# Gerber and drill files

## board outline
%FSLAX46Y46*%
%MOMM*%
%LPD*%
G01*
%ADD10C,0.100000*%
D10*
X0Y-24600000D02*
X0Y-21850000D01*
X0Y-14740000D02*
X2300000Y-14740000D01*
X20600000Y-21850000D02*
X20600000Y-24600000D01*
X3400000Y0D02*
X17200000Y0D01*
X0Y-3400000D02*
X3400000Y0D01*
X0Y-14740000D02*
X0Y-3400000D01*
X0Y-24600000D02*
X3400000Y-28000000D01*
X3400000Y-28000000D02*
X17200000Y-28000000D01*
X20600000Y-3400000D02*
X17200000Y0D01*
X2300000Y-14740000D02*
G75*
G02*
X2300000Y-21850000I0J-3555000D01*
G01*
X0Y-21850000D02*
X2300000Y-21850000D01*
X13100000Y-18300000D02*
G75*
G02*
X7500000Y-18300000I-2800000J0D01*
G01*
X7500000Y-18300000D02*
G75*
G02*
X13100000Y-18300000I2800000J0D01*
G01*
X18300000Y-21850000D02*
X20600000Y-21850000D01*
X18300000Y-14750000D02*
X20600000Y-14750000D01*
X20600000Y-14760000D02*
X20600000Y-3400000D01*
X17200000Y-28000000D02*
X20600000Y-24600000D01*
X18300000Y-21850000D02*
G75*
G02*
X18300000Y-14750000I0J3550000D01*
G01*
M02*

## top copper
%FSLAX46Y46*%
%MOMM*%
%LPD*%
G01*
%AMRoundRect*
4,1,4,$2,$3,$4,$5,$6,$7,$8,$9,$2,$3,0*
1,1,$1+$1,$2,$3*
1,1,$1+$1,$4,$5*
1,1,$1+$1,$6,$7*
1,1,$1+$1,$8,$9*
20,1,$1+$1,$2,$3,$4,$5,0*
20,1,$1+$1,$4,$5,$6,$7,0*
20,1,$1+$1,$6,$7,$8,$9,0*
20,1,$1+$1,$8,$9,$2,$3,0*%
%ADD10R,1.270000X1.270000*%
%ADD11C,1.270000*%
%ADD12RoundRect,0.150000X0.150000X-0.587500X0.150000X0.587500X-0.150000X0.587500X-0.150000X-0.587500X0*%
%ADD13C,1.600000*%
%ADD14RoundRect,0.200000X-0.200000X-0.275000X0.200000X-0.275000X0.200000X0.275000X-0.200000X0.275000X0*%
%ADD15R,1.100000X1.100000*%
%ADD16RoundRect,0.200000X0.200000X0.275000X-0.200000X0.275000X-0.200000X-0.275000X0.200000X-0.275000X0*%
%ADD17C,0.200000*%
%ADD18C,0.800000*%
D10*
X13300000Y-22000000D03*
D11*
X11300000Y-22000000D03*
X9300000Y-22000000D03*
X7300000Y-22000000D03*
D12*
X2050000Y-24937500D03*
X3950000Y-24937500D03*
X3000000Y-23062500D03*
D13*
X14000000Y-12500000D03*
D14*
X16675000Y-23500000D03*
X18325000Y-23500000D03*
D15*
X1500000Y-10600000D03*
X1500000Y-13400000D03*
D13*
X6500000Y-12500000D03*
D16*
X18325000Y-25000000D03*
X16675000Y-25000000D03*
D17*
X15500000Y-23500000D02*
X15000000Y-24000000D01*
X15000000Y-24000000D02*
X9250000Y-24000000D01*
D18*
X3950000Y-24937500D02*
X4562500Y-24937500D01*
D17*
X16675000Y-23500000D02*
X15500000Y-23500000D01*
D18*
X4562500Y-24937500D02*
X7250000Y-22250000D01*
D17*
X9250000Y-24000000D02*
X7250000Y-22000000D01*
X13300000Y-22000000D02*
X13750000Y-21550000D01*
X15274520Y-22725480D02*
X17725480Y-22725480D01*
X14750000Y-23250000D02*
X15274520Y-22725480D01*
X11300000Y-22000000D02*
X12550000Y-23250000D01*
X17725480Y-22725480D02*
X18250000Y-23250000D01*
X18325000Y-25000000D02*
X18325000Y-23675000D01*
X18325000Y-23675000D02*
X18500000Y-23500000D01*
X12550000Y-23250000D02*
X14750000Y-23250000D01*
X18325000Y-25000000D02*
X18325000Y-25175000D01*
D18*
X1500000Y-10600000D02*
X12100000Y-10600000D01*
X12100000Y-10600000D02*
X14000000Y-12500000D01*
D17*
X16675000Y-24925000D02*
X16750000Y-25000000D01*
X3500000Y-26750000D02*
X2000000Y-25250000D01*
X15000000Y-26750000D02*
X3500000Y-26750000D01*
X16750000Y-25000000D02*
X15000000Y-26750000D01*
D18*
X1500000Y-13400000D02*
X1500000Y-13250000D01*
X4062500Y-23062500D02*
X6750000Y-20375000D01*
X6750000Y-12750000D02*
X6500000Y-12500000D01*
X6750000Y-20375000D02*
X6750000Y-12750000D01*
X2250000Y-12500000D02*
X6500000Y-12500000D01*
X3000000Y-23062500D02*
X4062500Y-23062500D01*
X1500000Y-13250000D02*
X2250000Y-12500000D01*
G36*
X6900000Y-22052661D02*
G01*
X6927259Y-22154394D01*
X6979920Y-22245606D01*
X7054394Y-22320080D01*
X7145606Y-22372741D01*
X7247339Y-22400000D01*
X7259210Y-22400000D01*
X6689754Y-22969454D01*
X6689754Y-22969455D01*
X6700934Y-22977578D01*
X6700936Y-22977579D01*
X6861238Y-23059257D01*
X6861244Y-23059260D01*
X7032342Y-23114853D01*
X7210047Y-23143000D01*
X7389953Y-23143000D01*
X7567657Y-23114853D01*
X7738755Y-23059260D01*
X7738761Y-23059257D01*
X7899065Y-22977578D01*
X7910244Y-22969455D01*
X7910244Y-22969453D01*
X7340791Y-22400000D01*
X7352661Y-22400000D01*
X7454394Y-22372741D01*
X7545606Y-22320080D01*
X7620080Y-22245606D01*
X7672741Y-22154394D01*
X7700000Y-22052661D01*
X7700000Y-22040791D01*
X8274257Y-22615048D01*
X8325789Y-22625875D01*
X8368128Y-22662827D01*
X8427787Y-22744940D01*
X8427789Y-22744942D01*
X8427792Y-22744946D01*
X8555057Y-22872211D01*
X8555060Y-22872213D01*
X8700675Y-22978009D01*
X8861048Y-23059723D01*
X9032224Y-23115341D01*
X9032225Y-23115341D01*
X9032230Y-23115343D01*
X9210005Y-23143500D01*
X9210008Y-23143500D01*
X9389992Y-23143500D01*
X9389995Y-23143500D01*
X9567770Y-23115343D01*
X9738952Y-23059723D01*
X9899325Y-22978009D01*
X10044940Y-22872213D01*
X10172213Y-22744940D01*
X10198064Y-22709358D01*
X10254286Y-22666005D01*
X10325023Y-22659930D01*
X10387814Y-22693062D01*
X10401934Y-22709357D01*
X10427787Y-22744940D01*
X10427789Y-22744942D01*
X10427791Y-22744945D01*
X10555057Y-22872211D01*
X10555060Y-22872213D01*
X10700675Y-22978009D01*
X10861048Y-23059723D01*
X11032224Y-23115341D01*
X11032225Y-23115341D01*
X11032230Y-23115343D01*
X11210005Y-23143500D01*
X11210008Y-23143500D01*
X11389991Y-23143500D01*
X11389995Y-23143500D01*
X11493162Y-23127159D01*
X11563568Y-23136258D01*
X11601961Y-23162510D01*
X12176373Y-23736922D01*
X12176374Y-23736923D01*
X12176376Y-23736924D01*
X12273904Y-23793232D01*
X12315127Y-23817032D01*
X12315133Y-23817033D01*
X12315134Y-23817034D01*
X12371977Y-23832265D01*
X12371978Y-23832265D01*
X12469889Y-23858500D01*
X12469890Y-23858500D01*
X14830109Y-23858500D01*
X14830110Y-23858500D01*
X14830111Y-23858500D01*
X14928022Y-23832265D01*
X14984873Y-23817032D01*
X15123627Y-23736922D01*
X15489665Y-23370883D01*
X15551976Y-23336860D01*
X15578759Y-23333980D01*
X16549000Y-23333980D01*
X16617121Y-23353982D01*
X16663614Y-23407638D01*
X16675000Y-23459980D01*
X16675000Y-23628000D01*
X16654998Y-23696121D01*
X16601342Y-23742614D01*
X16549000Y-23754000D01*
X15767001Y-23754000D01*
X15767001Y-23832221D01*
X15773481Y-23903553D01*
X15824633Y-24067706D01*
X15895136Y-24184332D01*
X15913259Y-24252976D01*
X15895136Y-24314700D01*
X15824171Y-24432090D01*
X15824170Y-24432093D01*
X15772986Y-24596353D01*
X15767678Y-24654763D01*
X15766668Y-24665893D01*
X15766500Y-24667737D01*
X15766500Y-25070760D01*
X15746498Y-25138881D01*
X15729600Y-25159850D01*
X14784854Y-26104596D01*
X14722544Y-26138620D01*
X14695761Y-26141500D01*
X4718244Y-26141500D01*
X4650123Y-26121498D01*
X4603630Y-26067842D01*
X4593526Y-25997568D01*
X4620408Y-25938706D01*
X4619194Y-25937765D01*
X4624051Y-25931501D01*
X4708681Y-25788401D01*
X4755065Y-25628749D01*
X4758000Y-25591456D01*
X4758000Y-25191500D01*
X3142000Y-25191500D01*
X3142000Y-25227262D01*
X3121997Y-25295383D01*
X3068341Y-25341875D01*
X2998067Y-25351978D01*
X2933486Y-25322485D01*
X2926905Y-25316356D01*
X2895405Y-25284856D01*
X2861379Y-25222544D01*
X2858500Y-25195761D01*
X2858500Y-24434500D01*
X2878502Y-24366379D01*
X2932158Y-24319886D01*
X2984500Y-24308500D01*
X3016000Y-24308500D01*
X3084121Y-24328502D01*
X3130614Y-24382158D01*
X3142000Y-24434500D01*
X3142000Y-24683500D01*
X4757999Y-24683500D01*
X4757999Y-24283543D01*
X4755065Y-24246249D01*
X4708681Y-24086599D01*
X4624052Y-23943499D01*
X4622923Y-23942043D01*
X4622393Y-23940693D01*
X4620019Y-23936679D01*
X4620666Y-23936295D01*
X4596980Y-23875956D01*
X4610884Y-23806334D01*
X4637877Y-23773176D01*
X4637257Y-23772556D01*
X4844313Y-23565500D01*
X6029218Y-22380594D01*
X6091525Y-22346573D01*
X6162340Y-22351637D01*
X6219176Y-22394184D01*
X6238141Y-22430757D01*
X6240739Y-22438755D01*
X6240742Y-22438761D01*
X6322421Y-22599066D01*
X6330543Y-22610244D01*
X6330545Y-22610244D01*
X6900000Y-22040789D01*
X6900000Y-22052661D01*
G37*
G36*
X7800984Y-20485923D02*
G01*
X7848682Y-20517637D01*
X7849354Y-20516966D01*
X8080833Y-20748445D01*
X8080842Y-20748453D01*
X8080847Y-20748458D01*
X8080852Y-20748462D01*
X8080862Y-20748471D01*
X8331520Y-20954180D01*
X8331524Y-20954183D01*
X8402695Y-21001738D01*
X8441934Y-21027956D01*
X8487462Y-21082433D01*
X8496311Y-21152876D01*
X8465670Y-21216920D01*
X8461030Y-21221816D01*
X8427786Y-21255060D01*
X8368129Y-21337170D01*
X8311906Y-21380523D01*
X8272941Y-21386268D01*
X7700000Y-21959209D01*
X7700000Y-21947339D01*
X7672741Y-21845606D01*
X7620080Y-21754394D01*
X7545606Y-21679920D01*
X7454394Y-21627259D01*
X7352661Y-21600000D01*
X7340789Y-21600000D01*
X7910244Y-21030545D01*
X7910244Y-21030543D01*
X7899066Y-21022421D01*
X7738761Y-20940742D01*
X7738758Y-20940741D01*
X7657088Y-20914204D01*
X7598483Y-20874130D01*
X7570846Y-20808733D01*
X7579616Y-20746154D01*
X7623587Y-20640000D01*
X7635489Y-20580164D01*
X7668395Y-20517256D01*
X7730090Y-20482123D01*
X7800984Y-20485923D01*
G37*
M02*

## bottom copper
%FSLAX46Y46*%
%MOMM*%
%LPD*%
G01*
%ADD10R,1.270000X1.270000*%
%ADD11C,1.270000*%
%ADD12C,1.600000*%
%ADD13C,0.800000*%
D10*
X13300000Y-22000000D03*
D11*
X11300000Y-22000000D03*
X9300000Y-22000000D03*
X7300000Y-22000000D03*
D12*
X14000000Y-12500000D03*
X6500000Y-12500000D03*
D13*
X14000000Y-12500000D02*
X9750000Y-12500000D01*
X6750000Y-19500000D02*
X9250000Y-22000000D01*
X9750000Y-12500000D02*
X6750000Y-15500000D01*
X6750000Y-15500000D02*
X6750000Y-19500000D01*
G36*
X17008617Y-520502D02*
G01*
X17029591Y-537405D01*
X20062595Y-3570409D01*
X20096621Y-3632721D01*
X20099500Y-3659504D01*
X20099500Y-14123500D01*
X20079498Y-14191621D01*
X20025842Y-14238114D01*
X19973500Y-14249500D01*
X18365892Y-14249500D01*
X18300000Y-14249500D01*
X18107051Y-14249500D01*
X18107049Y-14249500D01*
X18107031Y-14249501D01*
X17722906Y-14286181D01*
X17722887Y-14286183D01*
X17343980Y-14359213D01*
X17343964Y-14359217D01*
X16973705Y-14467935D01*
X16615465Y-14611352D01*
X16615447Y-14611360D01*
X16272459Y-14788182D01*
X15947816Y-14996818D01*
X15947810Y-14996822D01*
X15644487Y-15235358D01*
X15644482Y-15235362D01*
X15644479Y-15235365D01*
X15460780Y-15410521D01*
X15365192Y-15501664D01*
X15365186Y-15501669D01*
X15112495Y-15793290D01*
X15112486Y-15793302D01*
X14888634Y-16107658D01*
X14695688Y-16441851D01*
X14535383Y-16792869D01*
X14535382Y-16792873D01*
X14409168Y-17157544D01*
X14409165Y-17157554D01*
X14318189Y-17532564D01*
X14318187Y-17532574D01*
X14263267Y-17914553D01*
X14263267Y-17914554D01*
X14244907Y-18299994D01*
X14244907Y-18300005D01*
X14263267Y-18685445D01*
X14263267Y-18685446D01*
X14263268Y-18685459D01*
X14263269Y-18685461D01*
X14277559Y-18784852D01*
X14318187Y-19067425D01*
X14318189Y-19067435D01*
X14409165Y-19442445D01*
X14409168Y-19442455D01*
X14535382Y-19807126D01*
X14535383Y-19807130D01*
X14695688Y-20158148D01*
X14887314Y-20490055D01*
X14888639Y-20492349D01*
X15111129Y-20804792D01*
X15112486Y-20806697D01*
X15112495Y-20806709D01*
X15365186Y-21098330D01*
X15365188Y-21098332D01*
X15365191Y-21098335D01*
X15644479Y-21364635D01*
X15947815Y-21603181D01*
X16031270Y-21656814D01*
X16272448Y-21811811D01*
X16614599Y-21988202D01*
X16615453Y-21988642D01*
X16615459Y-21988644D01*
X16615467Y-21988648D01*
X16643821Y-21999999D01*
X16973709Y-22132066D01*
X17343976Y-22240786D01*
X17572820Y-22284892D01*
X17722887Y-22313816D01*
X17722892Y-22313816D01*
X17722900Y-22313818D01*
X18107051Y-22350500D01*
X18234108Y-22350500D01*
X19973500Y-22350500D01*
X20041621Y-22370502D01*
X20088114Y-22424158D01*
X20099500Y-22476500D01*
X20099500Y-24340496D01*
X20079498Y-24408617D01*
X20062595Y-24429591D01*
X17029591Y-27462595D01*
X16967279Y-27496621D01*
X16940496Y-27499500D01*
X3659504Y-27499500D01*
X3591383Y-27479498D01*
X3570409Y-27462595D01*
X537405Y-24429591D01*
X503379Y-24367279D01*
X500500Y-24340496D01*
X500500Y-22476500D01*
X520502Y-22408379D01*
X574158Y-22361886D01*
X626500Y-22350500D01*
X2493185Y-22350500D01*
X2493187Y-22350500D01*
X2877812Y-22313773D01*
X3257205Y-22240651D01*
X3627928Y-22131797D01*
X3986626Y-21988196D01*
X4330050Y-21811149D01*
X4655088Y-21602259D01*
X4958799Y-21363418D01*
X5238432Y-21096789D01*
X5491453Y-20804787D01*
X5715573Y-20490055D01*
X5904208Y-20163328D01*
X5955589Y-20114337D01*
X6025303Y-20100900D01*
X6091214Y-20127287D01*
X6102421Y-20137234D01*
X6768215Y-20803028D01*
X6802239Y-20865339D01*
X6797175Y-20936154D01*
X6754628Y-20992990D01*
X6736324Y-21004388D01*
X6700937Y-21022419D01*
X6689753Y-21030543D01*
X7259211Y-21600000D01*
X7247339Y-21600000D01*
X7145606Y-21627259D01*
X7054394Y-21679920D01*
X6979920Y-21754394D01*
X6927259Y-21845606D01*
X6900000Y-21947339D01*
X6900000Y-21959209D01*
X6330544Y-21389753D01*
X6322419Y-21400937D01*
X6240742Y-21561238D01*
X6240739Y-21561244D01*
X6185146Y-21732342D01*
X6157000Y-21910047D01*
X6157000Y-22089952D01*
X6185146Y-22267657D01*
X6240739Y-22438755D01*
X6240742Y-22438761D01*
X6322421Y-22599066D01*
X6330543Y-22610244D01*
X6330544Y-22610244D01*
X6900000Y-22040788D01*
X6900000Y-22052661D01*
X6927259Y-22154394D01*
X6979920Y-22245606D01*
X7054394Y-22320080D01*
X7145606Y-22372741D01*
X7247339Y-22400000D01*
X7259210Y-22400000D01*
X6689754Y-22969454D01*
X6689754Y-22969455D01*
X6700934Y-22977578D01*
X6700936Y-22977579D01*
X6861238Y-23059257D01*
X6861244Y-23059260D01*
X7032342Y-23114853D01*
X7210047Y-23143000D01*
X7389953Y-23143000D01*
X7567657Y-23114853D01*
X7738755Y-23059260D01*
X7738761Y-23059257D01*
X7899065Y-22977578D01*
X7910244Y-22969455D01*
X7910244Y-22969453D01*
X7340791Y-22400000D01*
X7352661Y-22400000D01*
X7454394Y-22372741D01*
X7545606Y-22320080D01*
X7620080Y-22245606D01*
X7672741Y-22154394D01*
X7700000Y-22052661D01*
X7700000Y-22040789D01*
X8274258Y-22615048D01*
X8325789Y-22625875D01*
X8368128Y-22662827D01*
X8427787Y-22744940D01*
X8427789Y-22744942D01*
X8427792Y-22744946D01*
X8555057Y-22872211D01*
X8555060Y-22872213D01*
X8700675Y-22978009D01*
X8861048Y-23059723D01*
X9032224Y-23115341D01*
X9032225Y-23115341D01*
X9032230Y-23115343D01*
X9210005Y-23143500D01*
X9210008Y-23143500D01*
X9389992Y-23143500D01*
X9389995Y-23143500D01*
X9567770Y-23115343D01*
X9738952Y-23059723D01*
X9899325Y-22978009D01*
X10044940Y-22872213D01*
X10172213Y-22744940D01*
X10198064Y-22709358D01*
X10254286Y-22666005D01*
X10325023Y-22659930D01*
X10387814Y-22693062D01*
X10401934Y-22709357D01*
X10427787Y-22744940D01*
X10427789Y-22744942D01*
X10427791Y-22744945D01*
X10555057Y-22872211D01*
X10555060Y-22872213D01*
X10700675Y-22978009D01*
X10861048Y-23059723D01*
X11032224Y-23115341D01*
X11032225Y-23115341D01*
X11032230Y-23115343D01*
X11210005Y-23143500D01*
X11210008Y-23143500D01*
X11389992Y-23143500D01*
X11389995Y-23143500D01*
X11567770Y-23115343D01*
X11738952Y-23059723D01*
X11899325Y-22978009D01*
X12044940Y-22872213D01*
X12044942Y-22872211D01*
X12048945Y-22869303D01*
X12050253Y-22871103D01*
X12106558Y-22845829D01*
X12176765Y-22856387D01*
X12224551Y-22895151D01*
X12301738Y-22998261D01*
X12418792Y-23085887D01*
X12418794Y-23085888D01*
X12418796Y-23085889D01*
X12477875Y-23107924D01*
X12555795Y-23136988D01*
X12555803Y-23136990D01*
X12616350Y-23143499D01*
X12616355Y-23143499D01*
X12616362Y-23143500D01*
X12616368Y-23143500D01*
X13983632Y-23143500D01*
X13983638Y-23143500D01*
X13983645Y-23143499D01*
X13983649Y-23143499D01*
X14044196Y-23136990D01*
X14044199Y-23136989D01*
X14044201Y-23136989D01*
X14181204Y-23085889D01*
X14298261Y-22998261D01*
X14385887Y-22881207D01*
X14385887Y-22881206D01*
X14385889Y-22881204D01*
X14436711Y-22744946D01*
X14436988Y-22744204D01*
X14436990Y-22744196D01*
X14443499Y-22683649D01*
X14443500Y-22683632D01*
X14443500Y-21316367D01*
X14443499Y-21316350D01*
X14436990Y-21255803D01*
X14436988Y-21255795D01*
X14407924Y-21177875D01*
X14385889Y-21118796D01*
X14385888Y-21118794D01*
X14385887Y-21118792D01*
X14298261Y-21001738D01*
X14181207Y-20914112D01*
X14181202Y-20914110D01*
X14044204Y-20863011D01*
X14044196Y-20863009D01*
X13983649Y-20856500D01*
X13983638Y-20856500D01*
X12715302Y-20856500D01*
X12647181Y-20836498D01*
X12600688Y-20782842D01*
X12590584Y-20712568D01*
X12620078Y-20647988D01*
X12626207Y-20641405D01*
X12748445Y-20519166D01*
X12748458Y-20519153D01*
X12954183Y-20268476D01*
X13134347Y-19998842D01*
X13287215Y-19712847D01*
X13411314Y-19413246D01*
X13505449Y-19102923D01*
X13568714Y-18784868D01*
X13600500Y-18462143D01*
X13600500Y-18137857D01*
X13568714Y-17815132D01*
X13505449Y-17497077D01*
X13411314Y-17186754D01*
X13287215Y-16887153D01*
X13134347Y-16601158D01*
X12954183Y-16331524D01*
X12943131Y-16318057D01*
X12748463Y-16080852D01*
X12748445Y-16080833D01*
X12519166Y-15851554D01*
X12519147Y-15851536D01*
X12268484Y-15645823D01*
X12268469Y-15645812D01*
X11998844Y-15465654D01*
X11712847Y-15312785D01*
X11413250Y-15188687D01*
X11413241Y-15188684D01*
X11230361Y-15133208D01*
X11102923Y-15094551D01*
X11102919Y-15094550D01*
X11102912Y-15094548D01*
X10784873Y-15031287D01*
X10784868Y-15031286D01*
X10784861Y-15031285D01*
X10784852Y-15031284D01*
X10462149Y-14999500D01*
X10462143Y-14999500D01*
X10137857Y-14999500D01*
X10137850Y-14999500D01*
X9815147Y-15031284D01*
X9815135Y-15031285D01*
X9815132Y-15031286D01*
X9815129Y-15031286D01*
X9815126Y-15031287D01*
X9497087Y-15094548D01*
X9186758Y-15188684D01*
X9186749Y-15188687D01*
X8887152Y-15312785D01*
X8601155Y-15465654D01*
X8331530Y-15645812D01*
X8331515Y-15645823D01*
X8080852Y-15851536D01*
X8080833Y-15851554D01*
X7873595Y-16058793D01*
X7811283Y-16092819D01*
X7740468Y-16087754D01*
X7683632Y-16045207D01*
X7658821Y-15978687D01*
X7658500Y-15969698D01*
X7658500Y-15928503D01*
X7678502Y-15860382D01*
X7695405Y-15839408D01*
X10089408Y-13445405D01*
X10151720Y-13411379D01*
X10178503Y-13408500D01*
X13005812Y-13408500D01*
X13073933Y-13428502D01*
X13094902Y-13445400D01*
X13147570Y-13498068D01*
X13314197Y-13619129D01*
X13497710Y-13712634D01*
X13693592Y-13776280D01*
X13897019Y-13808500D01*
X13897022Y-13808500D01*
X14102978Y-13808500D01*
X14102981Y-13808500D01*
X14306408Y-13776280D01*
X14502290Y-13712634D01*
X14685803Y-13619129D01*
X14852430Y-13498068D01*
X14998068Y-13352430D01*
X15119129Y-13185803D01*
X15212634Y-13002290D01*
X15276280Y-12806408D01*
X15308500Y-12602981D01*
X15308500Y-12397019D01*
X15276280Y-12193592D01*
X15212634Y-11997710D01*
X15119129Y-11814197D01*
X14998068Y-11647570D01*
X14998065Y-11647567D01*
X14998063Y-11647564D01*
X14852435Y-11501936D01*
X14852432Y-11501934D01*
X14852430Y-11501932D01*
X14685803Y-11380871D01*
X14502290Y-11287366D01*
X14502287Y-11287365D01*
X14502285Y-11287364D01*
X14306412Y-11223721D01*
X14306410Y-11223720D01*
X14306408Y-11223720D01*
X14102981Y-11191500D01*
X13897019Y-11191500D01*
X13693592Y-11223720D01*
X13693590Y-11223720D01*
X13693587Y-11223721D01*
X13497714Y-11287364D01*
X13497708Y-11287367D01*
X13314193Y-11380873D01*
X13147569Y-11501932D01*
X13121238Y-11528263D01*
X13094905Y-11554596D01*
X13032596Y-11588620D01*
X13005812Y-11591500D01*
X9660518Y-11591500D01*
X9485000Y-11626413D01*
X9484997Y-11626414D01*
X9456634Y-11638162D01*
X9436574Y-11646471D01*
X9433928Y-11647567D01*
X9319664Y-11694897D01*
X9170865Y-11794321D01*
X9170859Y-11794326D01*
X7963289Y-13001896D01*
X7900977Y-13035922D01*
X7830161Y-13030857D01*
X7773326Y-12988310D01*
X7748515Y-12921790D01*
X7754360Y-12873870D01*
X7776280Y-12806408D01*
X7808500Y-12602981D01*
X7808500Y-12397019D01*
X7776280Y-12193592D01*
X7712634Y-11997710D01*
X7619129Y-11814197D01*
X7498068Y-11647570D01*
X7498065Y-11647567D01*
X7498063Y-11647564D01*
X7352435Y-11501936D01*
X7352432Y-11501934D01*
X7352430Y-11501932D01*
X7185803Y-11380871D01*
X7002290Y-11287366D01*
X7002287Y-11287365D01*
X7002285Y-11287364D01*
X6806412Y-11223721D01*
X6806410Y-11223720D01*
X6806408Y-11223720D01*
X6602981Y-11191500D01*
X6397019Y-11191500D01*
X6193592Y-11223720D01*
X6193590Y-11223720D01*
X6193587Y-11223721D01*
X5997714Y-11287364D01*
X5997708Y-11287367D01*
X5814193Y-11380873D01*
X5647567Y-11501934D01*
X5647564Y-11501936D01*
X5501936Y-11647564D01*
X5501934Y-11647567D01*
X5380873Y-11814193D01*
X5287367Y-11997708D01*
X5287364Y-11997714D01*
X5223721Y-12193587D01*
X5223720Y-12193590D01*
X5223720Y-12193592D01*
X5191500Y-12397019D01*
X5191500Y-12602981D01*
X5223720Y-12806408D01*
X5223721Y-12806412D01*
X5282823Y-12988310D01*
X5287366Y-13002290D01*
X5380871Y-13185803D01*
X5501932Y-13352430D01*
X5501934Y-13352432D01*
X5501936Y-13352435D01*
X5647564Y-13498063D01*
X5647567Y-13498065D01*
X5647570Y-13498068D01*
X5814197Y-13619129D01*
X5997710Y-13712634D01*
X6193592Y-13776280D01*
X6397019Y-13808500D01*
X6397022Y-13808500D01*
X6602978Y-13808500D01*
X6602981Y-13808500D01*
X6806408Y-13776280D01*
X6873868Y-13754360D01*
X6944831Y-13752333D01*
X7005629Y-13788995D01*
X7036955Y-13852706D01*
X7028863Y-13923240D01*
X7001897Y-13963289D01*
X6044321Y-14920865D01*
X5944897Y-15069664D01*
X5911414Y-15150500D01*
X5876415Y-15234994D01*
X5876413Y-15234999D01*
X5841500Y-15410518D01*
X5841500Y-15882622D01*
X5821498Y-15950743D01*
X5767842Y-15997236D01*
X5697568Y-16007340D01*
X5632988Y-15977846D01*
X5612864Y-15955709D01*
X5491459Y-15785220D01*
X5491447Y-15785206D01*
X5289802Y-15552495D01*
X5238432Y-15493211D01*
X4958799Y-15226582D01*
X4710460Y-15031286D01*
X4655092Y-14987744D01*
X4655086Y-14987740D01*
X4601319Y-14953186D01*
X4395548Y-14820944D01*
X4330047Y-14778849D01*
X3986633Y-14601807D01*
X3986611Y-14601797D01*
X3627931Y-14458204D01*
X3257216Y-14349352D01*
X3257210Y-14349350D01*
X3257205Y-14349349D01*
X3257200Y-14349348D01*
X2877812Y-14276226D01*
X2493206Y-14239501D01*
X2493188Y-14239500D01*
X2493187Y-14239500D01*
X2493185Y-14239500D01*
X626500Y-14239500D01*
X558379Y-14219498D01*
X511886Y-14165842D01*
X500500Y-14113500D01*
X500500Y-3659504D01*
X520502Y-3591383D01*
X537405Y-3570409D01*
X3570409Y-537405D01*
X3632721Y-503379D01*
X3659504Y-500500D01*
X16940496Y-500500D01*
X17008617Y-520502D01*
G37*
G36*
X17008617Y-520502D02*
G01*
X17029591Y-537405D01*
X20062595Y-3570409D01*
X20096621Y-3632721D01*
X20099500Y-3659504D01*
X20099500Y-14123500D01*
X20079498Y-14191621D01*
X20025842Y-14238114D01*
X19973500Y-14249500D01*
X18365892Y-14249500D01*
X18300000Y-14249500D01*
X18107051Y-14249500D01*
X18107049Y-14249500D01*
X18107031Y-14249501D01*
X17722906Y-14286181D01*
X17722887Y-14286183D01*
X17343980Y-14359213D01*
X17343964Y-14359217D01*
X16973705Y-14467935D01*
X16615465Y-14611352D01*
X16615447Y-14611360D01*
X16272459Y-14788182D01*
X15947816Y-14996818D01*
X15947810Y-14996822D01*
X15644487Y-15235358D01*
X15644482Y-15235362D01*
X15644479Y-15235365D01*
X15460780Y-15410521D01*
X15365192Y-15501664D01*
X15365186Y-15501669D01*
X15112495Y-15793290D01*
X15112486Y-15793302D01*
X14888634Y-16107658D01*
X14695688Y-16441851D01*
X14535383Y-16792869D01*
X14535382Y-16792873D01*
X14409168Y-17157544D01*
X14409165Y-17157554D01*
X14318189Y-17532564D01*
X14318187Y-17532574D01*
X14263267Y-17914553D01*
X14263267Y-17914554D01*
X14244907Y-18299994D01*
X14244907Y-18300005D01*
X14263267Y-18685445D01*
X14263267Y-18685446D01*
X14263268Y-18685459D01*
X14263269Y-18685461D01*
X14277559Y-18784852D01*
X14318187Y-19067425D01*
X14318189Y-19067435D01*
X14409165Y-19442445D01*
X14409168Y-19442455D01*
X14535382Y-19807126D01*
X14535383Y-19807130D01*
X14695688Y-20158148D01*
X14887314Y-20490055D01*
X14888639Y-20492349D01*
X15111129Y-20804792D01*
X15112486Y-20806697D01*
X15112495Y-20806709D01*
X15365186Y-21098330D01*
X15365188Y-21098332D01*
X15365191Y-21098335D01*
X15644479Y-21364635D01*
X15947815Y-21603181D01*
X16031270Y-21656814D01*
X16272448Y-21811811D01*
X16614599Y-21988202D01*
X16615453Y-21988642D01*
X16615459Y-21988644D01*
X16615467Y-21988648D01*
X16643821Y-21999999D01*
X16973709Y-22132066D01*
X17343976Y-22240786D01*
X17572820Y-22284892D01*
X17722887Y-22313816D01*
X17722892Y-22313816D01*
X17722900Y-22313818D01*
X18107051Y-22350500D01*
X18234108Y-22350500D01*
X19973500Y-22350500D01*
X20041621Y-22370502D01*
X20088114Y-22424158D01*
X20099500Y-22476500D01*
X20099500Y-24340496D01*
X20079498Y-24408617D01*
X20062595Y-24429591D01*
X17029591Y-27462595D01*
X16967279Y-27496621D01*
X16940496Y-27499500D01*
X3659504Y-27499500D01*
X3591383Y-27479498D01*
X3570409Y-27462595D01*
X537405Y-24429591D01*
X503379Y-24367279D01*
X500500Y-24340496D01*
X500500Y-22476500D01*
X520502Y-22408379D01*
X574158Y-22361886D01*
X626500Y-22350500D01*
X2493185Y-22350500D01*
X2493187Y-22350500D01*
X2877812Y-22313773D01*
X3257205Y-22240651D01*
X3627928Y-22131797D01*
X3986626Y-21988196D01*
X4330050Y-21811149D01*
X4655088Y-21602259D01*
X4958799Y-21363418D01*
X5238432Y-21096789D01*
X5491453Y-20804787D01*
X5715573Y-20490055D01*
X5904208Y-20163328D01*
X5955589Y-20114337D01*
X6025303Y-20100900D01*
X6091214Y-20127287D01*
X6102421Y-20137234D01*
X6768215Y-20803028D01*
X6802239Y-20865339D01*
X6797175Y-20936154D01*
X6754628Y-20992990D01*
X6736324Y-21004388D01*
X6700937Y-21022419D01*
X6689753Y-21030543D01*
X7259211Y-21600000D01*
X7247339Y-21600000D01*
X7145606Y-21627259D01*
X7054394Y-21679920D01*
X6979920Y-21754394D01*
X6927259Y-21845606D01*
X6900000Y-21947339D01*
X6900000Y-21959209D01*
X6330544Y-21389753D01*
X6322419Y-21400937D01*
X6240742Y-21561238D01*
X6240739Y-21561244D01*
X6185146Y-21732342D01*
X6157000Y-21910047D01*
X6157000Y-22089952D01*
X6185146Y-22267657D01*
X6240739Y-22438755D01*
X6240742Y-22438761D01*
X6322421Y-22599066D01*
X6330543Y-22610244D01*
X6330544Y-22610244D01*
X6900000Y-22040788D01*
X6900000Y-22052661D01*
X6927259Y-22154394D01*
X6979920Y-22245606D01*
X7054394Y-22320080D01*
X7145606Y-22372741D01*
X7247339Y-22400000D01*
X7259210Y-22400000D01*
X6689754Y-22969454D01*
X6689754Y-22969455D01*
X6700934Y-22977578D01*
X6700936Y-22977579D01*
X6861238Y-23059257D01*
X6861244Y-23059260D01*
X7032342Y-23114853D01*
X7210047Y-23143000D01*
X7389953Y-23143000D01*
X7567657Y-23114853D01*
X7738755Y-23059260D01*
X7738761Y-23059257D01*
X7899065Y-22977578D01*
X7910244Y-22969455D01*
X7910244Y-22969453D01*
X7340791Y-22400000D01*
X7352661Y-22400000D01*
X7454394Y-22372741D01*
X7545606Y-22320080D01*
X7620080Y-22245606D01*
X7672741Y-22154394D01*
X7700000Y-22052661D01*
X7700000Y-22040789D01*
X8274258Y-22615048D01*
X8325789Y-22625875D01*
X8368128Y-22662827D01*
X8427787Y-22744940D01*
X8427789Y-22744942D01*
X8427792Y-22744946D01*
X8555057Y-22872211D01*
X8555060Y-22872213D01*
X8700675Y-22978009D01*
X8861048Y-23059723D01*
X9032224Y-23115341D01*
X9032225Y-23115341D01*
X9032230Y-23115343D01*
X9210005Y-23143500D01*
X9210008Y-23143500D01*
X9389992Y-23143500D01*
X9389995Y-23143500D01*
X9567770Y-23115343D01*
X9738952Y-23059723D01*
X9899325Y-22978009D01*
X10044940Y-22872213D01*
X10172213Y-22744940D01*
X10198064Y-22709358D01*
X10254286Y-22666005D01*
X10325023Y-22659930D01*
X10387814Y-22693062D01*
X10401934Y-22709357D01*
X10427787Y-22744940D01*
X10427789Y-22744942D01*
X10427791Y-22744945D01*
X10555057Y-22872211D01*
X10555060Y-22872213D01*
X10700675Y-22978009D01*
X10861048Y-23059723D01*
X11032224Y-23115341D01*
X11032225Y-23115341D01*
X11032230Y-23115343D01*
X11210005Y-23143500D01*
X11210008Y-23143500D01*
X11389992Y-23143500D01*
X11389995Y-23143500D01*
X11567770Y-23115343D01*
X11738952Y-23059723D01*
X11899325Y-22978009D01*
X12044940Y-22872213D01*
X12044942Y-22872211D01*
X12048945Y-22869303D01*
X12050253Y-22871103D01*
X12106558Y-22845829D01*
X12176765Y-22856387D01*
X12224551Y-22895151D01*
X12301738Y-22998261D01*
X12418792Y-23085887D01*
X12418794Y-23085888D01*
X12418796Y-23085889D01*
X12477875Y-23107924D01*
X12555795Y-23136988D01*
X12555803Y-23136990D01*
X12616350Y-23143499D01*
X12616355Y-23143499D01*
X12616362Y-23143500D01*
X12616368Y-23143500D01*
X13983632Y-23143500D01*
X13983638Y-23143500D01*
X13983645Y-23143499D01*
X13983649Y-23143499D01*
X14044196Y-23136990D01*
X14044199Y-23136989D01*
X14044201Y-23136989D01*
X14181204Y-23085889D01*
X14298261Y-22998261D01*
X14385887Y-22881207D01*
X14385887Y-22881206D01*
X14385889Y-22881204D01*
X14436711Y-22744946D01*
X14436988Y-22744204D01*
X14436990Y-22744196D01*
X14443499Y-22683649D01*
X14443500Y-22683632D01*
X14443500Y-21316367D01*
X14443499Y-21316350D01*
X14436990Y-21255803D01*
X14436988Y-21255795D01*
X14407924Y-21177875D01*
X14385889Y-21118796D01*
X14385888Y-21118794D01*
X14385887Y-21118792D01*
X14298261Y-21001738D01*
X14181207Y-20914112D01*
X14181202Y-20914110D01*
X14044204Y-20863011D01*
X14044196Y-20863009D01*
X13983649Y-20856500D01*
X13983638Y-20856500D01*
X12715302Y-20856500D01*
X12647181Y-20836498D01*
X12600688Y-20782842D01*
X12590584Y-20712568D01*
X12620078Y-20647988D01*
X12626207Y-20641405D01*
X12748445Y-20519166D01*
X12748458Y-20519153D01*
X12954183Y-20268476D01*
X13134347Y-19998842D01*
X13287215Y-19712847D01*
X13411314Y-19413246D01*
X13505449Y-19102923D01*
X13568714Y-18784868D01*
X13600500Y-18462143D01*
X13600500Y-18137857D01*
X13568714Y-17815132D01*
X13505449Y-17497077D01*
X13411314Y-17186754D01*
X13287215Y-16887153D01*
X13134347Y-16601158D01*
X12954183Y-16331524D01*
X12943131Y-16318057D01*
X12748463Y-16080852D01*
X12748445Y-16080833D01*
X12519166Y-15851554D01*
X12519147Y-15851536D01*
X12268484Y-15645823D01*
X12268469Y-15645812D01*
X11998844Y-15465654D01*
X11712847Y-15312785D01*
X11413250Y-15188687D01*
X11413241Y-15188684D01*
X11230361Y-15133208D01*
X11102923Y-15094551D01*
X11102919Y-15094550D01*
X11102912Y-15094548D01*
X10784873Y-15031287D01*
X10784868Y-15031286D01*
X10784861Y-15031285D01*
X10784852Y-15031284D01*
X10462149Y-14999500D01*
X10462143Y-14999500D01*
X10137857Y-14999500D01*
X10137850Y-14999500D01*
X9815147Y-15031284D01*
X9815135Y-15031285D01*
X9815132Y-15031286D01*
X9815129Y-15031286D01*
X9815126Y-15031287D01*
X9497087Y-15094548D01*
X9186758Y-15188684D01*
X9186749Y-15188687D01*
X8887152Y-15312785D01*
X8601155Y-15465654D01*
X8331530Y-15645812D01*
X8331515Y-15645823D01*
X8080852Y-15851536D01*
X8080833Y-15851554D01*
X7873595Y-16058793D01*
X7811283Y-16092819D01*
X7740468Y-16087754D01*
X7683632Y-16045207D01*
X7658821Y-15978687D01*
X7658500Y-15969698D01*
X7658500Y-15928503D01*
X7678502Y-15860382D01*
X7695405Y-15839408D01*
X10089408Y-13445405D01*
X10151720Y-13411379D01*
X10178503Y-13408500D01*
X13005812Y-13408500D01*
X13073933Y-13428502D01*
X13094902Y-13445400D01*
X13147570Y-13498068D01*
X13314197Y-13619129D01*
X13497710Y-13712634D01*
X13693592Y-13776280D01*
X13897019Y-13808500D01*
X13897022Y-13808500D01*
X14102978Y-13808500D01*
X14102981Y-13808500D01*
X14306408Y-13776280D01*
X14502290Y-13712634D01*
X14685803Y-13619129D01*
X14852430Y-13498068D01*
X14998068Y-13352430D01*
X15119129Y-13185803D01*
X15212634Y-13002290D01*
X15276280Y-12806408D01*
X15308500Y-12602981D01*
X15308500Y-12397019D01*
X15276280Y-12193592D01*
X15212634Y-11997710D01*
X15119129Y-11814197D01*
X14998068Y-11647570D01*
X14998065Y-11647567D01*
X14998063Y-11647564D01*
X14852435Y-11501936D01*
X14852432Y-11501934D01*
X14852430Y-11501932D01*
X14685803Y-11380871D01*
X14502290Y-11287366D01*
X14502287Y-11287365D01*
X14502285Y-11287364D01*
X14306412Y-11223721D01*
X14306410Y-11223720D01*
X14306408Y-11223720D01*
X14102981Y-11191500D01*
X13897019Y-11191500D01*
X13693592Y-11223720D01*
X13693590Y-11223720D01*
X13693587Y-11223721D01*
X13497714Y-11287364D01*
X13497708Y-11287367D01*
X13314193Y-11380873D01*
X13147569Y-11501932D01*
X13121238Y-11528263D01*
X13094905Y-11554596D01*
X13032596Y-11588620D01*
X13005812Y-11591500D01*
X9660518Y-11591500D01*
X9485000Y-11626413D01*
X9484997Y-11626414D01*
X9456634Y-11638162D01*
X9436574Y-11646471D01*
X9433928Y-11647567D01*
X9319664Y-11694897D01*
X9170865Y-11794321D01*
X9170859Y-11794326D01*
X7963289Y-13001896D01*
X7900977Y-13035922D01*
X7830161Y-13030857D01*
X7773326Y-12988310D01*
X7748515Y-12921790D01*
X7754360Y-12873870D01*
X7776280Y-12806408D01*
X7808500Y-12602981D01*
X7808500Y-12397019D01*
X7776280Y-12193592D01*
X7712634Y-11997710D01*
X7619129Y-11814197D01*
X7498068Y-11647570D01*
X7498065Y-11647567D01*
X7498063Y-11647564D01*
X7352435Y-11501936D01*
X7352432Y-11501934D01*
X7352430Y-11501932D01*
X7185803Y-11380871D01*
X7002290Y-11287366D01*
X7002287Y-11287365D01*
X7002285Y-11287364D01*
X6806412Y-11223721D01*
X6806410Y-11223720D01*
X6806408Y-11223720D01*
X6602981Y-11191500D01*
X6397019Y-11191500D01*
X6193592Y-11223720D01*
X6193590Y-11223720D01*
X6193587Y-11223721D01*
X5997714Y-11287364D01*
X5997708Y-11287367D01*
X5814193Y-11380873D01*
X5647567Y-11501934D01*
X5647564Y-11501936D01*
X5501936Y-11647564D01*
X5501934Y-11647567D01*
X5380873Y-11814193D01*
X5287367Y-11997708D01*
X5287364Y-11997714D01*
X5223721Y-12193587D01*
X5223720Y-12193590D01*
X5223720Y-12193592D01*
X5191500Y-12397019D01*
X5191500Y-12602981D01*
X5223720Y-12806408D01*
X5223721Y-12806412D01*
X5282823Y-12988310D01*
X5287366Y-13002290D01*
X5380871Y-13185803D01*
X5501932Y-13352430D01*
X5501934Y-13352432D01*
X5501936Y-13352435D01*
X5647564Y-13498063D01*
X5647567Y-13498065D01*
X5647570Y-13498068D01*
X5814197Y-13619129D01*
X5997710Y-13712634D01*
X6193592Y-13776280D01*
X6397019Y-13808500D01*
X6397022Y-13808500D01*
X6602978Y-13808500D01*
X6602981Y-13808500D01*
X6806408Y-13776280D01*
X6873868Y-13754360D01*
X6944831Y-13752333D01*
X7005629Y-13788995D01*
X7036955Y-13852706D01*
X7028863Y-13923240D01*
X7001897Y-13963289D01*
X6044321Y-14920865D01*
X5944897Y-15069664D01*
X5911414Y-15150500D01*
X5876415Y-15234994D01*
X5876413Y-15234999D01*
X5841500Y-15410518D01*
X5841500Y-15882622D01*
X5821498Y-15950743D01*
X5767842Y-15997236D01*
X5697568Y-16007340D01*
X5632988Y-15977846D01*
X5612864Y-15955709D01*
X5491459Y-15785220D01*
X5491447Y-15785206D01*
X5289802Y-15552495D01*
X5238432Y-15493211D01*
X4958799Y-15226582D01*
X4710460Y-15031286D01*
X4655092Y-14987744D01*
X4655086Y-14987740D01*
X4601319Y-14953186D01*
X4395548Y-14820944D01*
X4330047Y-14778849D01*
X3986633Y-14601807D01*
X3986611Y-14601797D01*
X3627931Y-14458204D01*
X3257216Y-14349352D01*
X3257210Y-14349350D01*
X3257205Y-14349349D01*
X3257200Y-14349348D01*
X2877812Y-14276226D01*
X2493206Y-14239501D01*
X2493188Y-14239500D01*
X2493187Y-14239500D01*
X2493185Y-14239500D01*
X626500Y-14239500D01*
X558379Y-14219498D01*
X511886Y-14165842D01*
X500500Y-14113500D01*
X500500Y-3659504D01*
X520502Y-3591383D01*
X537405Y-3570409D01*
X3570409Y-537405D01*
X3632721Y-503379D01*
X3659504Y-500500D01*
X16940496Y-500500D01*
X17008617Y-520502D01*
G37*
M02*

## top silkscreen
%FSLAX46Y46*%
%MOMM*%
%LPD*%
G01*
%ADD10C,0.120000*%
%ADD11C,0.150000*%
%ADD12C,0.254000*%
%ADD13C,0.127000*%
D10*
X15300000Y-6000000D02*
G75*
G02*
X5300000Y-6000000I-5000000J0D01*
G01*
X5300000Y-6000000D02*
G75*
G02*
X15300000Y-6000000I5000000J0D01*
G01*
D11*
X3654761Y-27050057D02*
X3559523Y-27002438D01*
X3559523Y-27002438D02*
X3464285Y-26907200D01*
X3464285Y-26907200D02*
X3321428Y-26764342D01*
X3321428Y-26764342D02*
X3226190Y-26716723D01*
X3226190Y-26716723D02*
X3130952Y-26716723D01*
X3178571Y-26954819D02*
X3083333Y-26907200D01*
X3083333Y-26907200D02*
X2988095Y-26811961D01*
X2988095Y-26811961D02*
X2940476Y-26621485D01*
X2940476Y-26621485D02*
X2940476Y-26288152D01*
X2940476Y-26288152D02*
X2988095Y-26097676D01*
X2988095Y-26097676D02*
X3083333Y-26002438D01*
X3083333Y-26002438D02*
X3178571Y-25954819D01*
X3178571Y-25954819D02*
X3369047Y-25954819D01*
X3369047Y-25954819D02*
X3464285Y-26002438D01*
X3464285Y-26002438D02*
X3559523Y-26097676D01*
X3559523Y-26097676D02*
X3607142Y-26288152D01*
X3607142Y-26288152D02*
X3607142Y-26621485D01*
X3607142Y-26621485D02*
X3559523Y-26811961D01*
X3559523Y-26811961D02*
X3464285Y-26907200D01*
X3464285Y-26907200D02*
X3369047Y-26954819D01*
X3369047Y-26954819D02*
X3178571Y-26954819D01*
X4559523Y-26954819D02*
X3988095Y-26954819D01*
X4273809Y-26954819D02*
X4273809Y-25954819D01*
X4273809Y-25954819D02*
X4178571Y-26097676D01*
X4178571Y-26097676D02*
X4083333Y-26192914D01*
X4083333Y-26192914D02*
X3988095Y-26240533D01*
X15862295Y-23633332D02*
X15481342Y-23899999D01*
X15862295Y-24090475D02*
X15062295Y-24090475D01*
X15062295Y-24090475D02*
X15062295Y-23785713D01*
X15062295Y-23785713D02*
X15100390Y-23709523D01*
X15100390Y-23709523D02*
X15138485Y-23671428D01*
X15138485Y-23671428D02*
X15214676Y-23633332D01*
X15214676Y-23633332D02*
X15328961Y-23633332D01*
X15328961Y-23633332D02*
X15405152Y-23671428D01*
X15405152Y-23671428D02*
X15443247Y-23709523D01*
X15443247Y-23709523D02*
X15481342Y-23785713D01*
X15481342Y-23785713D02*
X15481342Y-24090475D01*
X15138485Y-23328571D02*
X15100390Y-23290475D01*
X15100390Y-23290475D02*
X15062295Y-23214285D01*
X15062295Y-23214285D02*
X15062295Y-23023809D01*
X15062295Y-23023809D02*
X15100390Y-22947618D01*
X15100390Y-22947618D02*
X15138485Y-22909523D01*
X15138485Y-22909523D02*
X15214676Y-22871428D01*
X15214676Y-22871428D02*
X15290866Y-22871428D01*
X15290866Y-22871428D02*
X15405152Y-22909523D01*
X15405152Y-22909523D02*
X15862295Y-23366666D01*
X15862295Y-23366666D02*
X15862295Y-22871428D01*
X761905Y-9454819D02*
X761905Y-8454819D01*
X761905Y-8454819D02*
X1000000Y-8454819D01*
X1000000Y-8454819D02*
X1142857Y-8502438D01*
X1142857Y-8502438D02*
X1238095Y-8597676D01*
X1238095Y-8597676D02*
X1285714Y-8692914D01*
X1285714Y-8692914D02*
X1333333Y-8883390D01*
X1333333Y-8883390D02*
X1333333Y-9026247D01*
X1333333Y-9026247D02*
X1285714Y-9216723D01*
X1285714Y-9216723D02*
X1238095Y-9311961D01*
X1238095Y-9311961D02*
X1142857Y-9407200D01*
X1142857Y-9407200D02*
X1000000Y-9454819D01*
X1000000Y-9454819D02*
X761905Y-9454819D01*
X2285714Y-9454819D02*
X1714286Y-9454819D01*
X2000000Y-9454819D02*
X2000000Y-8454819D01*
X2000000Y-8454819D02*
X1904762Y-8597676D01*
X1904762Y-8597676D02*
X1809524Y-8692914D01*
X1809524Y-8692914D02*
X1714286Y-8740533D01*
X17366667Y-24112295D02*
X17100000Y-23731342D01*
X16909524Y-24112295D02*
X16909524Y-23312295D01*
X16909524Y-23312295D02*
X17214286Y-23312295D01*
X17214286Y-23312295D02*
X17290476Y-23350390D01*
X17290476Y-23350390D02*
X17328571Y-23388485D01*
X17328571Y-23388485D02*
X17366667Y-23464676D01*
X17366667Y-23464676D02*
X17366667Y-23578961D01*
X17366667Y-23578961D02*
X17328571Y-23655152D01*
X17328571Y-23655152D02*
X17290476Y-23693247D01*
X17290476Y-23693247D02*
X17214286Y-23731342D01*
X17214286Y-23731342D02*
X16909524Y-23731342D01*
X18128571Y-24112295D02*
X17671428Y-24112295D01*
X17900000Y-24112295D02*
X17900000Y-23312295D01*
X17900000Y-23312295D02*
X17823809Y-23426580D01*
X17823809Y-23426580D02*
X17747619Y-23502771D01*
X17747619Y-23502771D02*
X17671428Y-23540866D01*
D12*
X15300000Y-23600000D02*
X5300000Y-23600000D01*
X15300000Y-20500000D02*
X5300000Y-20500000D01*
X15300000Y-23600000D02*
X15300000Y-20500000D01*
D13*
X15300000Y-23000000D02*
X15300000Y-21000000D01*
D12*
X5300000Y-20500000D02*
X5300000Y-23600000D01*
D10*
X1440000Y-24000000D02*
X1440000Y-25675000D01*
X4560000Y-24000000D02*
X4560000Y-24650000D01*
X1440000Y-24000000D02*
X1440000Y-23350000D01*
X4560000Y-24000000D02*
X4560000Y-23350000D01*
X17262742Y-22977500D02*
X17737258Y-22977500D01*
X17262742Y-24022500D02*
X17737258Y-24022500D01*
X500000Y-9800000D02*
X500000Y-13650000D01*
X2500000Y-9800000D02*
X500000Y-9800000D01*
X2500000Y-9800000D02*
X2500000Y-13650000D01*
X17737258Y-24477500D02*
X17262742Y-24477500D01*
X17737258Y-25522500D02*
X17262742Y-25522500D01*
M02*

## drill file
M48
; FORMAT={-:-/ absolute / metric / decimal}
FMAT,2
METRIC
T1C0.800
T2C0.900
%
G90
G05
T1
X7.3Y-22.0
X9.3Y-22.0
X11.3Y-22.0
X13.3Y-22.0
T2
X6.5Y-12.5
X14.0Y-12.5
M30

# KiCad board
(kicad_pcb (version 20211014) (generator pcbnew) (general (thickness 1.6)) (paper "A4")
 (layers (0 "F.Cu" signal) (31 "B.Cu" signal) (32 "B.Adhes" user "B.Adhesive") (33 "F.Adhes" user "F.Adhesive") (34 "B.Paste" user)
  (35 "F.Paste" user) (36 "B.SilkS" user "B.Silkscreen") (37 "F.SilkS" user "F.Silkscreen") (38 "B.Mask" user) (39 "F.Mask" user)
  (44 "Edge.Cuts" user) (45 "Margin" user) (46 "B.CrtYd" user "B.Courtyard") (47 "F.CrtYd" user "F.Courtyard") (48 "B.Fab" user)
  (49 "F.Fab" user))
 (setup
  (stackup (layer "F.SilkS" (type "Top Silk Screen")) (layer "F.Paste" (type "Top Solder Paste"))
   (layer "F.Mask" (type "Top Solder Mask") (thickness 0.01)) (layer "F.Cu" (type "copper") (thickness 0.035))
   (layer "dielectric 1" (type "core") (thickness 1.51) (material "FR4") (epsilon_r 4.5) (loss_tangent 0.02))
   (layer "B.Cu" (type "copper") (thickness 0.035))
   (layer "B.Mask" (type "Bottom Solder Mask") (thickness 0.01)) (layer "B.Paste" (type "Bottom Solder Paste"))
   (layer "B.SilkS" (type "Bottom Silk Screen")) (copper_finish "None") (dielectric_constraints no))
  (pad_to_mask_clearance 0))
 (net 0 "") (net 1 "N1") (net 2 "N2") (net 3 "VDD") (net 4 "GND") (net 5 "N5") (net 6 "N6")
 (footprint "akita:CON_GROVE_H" (layer "F.Cu") (at 10.3 22 180)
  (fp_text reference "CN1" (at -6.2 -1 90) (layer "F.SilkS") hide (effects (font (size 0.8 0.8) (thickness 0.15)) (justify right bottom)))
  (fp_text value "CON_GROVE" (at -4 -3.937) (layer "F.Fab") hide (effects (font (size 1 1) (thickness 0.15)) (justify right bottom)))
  (fp_line (start -5 -1.6) (end 5 -1.6) (layer "F.SilkS") (width 0.254))
  (fp_line (start -5 1.5) (end 5 1.5) (layer "F.SilkS") (width 0.254))
  (fp_line (start -5 -1.6) (end -5 1.5) (layer "F.SilkS") (width 0.254))
  (fp_line (start -5 -1) (end -5 1) (layer "F.SilkS") (width 0.127))
  (fp_line (start 5 1.5) (end 5 -1.6) (layer "F.SilkS") (width 0.254))
  (pad "1" thru_hole rect (at -3 0 180) (size 1.27 1.27) (drill 0.8) (layers *.Cu *.Mask) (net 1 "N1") (solder_mask_margin 0.1016))
  (pad "2" thru_hole circle (at -1 0 180) (size 1.27 1.27) (drill 0.8) (layers *.Cu *.Mask) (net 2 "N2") (solder_mask_margin 0.1016))
  (pad "3" thru_hole circle (at 1 0 180) (size 1.27 1.27) (drill 0.8) (layers *.Cu *.Mask) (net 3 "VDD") (solder_mask_margin 0.1016))
  (pad "4" thru_hole circle (at 3 0 180) (size 1.27 1.27) (drill 0.8) (layers *.Cu *.Mask) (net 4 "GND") (solder_mask_margin 0.1016)))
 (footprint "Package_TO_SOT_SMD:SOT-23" (layer "F.Cu") (at 3 24 90)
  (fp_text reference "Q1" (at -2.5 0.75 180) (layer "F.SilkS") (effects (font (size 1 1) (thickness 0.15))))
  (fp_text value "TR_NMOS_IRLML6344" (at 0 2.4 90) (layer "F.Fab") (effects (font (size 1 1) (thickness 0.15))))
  (fp_line (start 0 -1.56) (end -1.675 -1.56) (layer "F.SilkS") (width 0.12))
  (fp_line (start 0 1.56) (end -0.65 1.56) (layer "F.SilkS") (width 0.12))
  (fp_line (start 0 -1.56) (end 0.65 -1.56) (layer "F.SilkS") (width 0.12))
  (fp_line (start 0 1.56) (end 0.65 1.56) (layer "F.SilkS") (width 0.12))
  (pad "1" smd roundrect locked (at -0.9375 -0.95 90) (size 1.475 0.6) (layers "F.Cu" "F.Paste" "F.Mask") (roundrect_rratio 0.25)
   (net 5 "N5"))
  (pad "2" smd roundrect locked (at -0.9375 0.95 90) (size 1.475 0.6) (layers "F.Cu" "F.Paste" "F.Mask") (roundrect_rratio 0.25)
   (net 4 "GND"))
  (pad "3" smd roundrect locked (at 0.9375 0 90) (size 1.475 0.6) (layers "F.Cu" "F.Paste" "F.Mask") (roundrect_rratio 0.25) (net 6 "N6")))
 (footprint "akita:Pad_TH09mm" (layer "F.Cu") (at 14 12.5 11)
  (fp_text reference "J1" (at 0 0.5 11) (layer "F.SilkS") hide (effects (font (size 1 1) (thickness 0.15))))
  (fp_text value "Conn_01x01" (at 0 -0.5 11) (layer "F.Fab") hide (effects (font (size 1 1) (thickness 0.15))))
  (pad "1" thru_hole circle locked (at 0 0 11) (size 1.6 1.6) (drill 0.9) (layers *.Cu *.Mask) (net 3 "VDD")))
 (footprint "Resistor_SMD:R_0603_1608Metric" (layer "F.Cu") (at 17.5 23.5)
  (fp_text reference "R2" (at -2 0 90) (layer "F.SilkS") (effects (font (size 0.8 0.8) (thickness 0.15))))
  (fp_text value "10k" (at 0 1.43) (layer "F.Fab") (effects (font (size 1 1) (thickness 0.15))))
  (fp_line (start -0.237258 -0.5225) (end 0.237258 -0.5225) (layer "F.SilkS") (width 0.12))
  (fp_line (start -0.237258 0.5225) (end 0.237258 0.5225) (layer "F.SilkS") (width 0.12))
  (pad "1" smd roundrect locked (at -0.825 0) (size 0.8 0.95) (layers "F.Cu" "F.Paste" "F.Mask") (roundrect_rratio 0.25) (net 4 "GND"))
  (pad "2" smd roundrect locked (at 0.825 0) (size 0.8 0.95) (layers "F.Cu" "F.Paste" "F.Mask") (roundrect_rratio 0.25) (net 2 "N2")))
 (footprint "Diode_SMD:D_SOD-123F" (layer "F.Cu") (at 1.5 12 -90)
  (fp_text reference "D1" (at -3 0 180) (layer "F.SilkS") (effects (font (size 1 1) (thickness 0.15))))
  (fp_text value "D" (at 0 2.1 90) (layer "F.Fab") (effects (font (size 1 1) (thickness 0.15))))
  (fp_line (start -2.2 1) (end 1.65 1) (layer "F.SilkS") (width 0.12))
  (fp_line (start -2.2 -1) (end -2.2 1) (layer "F.SilkS") (width 0.12))
  (fp_line (start -2.2 -1) (end 1.65 -1) (layer "F.SilkS") (width 0.12))
  (pad "1" smd rect locked (at -1.4 0 270) (size 1.1 1.1) (layers "F.Cu" "F.Paste" "F.Mask") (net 3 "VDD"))
  (pad "2" smd rect locked (at 1.4 0 270) (size 1.1 1.1) (layers "F.Cu" "F.Paste" "F.Mask") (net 6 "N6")))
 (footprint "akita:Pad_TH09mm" (layer "F.Cu") (at 6.5 12.5)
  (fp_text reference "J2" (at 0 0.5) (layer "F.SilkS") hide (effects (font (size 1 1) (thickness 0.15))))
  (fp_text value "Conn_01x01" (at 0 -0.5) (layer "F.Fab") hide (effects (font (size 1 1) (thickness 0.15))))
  (pad "1" thru_hole circle locked (at 0 0) (size 1.6 1.6) (drill 0.9) (layers *.Cu *.Mask) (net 6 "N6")))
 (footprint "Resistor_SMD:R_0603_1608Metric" (layer "F.Cu") (at 17.5 25 180)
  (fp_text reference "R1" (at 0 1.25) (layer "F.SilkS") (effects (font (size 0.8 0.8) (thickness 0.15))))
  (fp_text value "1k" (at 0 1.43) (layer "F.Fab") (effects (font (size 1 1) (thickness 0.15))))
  (fp_line (start -0.237258 0.5225) (end 0.237258 0.5225) (layer "F.SilkS") (width 0.12))
  (fp_line (start -0.237258 -0.5225) (end 0.237258 -0.5225) (layer "F.SilkS") (width 0.12))
  (pad "1" smd roundrect locked (at -0.825 0 180) (size 0.8 0.95) (layers "F.Cu" "F.Paste" "F.Mask") (roundrect_rratio 0.25) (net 2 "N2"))
  (pad "2" smd roundrect locked (at 0.825 0 180) (size 0.8 0.95) (layers "F.Cu" "F.Paste" "F.Mask") (roundrect_rratio 0.25) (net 5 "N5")))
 (gr_circle (center 10.3 6) (end 15.3 6) (layer "F.SilkS") (width 0.12) (fill none))
 (gr_line (start 0 24.6) (end 0 21.85) (layer "Edge.Cuts") (width 0.1))
 (gr_line (start 0 14.74) (end 2.3 14.74) (layer "Edge.Cuts") (width 0.1))
 (gr_line (start 20.6 21.85) (end 20.6 24.6) (layer "Edge.Cuts") (width 0.1))
 (gr_line (start 3.4 0) (end 17.2 0) (layer "Edge.Cuts") (width 0.1))
 (gr_line (start 0 3.4) (end 3.4 0) (layer "Edge.Cuts") (width 0.1))
 (gr_line (start 0 14.74) (end 0 3.4) (layer "Edge.Cuts") (width 0.1))
 (gr_line (start 0 24.6) (end 3.4 28) (layer "Edge.Cuts") (width 0.1))
 (gr_line (start 3.4 28) (end 17.2 28) (layer "Edge.Cuts") (width 0.1))
 (gr_line (start 20.6 3.4) (end 17.2 0) (layer "Edge.Cuts") (width 0.1))
 (gr_arc (start 2.3 14.74) (mid 5.855 18.295) (end 2.3 21.85) (layer "Edge.Cuts") (width 0.1))
 (gr_line (start 0 21.85) (end 2.3 21.85) (layer "Edge.Cuts") (width 0.1))
 (gr_circle (center 10.3 18.3) (end 13.1 18.3) (layer "Edge.Cuts") (width 0.1) (fill none))
 (gr_line (start 18.3 21.85) (end 20.6 21.85) (layer "Edge.Cuts") (width 0.1))
 (gr_line (start 18.3 14.75) (end 20.6 14.75) (layer "Edge.Cuts") (width 0.1))
 (gr_line (start 20.6 14.76) (end 20.6 3.4) (layer "Edge.Cuts") (width 0.1))
 (gr_line (start 17.2 28) (end 20.6 24.6) (layer "Edge.Cuts") (width 0.1))
 (gr_arc (start 18.3 21.85) (mid 14.75 18.3) (end 18.3 14.75) (layer "Edge.Cuts") (width 0.1))
 (segment (start 15.5 23.5) (end 15 24) (width 0.2) (layer "F.Cu") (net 4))
 (segment (start 15 24) (end 9.25 24) (width 0.2) (layer "F.Cu") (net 4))
 (segment (start 3.95 24.9375) (end 4.5625 24.9375) (width 0.8) (layer "F.Cu") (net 4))
 (segment (start 16.675 23.5) (end 15.5 23.5) (width 0.2) (layer "F.Cu") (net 4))
 (segment (start 4.5625 24.9375) (end 7.25 22.25) (width 0.8) (layer "F.Cu") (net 4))
 (segment (start 9.25 24) (end 7.25 22) (width 0.2) (layer "F.Cu") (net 4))
 (segment (start 13.3 22) (end 13.75 21.55) (width 0.2) (layer "F.Cu") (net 1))
 (segment (start 15.27452 22.72548) (end 17.72548 22.72548) (width 0.2) (layer "F.Cu") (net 2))
 (segment (start 14.75 23.25) (end 15.27452 22.72548) (width 0.2) (layer "F.Cu") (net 2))
 (segment (start 11.3 22) (end 12.55 23.25) (width 0.2) (layer "F.Cu") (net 2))
 (segment (start 17.72548 22.72548) (end 18.25 23.25) (width 0.2) (layer "F.Cu") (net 2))
 (segment (start 18.325 25) (end 18.325 23.675) (width 0.2) (layer "F.Cu") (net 2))
 (segment (start 18.325 23.675) (end 18.5 23.5) (width 0.2) (layer "F.Cu") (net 2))
 (segment (start 12.55 23.25) (end 14.75 23.25) (width 0.2) (layer "F.Cu") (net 2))
 (segment (start 18.325 25) (end 18.325 25.175) (width 0.2) (layer "F.Cu") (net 2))
 (segment (start 1.5 10.6) (end 12.1 10.6) (width 0.8) (layer "F.Cu") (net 3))
 (segment (start 12.1 10.6) (end 14 12.5) (width 0.8) (layer "F.Cu") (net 3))
 (segment (start 14 12.5) (end 9.75 12.5) (width 0.8) (layer "B.Cu") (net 3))
 (segment (start 6.75 19.5) (end 9.25 22) (width 0.8) (layer "B.Cu") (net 3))
 (segment (start 9.75 12.5) (end 6.75 15.5) (width 0.8) (layer "B.Cu") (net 3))
 (segment (start 6.75 15.5) (end 6.75 19.5) (width 0.8) (layer "B.Cu") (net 3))
 (segment (start 16.675 24.925) (end 16.75 25) (width 0.2) (layer "F.Cu") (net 5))
 (segment (start 3.5 26.75) (end 2 25.25) (width 0.2) (layer "F.Cu") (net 5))
 (segment (start 15 26.75) (end 3.5 26.75) (width 0.2) (layer "F.Cu") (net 5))
 (segment (start 16.75 25) (end 15 26.75) (width 0.2) (layer "F.Cu") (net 5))
 (segment (start 1.5 13.4) (end 1.5 13.25) (width 0.8) (layer "F.Cu") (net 6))
 (segment (start 4.0625 23.0625) (end 6.75 20.375) (width 0.8) (layer "F.Cu") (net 6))
 (segment (start 6.75 12.75) (end 6.5 12.5) (width 0.8) (layer "F.Cu") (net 6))
 (segment (start 6.75 20.375) (end 6.75 12.75) (width 0.8) (layer "F.Cu") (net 6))
 (segment (start 2.25 12.5) (end 6.5 12.5) (width 0.8) (layer "F.Cu") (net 6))
 (segment (start 3 23.0625) (end 4.0625 23.0625) (width 0.8) (layer "F.Cu") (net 6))
 (segment (start 1.5 13.25) (end 2.25 12.5) (width 0.8) (layer "F.Cu") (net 6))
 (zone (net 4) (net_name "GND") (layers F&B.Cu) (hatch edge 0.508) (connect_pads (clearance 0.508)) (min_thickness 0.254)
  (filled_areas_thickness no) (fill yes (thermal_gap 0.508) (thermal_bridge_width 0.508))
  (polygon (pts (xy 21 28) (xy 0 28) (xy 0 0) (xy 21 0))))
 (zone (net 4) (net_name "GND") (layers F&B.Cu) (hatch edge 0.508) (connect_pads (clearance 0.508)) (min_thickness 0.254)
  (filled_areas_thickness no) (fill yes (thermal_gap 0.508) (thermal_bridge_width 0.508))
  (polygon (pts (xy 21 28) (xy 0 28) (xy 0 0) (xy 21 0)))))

